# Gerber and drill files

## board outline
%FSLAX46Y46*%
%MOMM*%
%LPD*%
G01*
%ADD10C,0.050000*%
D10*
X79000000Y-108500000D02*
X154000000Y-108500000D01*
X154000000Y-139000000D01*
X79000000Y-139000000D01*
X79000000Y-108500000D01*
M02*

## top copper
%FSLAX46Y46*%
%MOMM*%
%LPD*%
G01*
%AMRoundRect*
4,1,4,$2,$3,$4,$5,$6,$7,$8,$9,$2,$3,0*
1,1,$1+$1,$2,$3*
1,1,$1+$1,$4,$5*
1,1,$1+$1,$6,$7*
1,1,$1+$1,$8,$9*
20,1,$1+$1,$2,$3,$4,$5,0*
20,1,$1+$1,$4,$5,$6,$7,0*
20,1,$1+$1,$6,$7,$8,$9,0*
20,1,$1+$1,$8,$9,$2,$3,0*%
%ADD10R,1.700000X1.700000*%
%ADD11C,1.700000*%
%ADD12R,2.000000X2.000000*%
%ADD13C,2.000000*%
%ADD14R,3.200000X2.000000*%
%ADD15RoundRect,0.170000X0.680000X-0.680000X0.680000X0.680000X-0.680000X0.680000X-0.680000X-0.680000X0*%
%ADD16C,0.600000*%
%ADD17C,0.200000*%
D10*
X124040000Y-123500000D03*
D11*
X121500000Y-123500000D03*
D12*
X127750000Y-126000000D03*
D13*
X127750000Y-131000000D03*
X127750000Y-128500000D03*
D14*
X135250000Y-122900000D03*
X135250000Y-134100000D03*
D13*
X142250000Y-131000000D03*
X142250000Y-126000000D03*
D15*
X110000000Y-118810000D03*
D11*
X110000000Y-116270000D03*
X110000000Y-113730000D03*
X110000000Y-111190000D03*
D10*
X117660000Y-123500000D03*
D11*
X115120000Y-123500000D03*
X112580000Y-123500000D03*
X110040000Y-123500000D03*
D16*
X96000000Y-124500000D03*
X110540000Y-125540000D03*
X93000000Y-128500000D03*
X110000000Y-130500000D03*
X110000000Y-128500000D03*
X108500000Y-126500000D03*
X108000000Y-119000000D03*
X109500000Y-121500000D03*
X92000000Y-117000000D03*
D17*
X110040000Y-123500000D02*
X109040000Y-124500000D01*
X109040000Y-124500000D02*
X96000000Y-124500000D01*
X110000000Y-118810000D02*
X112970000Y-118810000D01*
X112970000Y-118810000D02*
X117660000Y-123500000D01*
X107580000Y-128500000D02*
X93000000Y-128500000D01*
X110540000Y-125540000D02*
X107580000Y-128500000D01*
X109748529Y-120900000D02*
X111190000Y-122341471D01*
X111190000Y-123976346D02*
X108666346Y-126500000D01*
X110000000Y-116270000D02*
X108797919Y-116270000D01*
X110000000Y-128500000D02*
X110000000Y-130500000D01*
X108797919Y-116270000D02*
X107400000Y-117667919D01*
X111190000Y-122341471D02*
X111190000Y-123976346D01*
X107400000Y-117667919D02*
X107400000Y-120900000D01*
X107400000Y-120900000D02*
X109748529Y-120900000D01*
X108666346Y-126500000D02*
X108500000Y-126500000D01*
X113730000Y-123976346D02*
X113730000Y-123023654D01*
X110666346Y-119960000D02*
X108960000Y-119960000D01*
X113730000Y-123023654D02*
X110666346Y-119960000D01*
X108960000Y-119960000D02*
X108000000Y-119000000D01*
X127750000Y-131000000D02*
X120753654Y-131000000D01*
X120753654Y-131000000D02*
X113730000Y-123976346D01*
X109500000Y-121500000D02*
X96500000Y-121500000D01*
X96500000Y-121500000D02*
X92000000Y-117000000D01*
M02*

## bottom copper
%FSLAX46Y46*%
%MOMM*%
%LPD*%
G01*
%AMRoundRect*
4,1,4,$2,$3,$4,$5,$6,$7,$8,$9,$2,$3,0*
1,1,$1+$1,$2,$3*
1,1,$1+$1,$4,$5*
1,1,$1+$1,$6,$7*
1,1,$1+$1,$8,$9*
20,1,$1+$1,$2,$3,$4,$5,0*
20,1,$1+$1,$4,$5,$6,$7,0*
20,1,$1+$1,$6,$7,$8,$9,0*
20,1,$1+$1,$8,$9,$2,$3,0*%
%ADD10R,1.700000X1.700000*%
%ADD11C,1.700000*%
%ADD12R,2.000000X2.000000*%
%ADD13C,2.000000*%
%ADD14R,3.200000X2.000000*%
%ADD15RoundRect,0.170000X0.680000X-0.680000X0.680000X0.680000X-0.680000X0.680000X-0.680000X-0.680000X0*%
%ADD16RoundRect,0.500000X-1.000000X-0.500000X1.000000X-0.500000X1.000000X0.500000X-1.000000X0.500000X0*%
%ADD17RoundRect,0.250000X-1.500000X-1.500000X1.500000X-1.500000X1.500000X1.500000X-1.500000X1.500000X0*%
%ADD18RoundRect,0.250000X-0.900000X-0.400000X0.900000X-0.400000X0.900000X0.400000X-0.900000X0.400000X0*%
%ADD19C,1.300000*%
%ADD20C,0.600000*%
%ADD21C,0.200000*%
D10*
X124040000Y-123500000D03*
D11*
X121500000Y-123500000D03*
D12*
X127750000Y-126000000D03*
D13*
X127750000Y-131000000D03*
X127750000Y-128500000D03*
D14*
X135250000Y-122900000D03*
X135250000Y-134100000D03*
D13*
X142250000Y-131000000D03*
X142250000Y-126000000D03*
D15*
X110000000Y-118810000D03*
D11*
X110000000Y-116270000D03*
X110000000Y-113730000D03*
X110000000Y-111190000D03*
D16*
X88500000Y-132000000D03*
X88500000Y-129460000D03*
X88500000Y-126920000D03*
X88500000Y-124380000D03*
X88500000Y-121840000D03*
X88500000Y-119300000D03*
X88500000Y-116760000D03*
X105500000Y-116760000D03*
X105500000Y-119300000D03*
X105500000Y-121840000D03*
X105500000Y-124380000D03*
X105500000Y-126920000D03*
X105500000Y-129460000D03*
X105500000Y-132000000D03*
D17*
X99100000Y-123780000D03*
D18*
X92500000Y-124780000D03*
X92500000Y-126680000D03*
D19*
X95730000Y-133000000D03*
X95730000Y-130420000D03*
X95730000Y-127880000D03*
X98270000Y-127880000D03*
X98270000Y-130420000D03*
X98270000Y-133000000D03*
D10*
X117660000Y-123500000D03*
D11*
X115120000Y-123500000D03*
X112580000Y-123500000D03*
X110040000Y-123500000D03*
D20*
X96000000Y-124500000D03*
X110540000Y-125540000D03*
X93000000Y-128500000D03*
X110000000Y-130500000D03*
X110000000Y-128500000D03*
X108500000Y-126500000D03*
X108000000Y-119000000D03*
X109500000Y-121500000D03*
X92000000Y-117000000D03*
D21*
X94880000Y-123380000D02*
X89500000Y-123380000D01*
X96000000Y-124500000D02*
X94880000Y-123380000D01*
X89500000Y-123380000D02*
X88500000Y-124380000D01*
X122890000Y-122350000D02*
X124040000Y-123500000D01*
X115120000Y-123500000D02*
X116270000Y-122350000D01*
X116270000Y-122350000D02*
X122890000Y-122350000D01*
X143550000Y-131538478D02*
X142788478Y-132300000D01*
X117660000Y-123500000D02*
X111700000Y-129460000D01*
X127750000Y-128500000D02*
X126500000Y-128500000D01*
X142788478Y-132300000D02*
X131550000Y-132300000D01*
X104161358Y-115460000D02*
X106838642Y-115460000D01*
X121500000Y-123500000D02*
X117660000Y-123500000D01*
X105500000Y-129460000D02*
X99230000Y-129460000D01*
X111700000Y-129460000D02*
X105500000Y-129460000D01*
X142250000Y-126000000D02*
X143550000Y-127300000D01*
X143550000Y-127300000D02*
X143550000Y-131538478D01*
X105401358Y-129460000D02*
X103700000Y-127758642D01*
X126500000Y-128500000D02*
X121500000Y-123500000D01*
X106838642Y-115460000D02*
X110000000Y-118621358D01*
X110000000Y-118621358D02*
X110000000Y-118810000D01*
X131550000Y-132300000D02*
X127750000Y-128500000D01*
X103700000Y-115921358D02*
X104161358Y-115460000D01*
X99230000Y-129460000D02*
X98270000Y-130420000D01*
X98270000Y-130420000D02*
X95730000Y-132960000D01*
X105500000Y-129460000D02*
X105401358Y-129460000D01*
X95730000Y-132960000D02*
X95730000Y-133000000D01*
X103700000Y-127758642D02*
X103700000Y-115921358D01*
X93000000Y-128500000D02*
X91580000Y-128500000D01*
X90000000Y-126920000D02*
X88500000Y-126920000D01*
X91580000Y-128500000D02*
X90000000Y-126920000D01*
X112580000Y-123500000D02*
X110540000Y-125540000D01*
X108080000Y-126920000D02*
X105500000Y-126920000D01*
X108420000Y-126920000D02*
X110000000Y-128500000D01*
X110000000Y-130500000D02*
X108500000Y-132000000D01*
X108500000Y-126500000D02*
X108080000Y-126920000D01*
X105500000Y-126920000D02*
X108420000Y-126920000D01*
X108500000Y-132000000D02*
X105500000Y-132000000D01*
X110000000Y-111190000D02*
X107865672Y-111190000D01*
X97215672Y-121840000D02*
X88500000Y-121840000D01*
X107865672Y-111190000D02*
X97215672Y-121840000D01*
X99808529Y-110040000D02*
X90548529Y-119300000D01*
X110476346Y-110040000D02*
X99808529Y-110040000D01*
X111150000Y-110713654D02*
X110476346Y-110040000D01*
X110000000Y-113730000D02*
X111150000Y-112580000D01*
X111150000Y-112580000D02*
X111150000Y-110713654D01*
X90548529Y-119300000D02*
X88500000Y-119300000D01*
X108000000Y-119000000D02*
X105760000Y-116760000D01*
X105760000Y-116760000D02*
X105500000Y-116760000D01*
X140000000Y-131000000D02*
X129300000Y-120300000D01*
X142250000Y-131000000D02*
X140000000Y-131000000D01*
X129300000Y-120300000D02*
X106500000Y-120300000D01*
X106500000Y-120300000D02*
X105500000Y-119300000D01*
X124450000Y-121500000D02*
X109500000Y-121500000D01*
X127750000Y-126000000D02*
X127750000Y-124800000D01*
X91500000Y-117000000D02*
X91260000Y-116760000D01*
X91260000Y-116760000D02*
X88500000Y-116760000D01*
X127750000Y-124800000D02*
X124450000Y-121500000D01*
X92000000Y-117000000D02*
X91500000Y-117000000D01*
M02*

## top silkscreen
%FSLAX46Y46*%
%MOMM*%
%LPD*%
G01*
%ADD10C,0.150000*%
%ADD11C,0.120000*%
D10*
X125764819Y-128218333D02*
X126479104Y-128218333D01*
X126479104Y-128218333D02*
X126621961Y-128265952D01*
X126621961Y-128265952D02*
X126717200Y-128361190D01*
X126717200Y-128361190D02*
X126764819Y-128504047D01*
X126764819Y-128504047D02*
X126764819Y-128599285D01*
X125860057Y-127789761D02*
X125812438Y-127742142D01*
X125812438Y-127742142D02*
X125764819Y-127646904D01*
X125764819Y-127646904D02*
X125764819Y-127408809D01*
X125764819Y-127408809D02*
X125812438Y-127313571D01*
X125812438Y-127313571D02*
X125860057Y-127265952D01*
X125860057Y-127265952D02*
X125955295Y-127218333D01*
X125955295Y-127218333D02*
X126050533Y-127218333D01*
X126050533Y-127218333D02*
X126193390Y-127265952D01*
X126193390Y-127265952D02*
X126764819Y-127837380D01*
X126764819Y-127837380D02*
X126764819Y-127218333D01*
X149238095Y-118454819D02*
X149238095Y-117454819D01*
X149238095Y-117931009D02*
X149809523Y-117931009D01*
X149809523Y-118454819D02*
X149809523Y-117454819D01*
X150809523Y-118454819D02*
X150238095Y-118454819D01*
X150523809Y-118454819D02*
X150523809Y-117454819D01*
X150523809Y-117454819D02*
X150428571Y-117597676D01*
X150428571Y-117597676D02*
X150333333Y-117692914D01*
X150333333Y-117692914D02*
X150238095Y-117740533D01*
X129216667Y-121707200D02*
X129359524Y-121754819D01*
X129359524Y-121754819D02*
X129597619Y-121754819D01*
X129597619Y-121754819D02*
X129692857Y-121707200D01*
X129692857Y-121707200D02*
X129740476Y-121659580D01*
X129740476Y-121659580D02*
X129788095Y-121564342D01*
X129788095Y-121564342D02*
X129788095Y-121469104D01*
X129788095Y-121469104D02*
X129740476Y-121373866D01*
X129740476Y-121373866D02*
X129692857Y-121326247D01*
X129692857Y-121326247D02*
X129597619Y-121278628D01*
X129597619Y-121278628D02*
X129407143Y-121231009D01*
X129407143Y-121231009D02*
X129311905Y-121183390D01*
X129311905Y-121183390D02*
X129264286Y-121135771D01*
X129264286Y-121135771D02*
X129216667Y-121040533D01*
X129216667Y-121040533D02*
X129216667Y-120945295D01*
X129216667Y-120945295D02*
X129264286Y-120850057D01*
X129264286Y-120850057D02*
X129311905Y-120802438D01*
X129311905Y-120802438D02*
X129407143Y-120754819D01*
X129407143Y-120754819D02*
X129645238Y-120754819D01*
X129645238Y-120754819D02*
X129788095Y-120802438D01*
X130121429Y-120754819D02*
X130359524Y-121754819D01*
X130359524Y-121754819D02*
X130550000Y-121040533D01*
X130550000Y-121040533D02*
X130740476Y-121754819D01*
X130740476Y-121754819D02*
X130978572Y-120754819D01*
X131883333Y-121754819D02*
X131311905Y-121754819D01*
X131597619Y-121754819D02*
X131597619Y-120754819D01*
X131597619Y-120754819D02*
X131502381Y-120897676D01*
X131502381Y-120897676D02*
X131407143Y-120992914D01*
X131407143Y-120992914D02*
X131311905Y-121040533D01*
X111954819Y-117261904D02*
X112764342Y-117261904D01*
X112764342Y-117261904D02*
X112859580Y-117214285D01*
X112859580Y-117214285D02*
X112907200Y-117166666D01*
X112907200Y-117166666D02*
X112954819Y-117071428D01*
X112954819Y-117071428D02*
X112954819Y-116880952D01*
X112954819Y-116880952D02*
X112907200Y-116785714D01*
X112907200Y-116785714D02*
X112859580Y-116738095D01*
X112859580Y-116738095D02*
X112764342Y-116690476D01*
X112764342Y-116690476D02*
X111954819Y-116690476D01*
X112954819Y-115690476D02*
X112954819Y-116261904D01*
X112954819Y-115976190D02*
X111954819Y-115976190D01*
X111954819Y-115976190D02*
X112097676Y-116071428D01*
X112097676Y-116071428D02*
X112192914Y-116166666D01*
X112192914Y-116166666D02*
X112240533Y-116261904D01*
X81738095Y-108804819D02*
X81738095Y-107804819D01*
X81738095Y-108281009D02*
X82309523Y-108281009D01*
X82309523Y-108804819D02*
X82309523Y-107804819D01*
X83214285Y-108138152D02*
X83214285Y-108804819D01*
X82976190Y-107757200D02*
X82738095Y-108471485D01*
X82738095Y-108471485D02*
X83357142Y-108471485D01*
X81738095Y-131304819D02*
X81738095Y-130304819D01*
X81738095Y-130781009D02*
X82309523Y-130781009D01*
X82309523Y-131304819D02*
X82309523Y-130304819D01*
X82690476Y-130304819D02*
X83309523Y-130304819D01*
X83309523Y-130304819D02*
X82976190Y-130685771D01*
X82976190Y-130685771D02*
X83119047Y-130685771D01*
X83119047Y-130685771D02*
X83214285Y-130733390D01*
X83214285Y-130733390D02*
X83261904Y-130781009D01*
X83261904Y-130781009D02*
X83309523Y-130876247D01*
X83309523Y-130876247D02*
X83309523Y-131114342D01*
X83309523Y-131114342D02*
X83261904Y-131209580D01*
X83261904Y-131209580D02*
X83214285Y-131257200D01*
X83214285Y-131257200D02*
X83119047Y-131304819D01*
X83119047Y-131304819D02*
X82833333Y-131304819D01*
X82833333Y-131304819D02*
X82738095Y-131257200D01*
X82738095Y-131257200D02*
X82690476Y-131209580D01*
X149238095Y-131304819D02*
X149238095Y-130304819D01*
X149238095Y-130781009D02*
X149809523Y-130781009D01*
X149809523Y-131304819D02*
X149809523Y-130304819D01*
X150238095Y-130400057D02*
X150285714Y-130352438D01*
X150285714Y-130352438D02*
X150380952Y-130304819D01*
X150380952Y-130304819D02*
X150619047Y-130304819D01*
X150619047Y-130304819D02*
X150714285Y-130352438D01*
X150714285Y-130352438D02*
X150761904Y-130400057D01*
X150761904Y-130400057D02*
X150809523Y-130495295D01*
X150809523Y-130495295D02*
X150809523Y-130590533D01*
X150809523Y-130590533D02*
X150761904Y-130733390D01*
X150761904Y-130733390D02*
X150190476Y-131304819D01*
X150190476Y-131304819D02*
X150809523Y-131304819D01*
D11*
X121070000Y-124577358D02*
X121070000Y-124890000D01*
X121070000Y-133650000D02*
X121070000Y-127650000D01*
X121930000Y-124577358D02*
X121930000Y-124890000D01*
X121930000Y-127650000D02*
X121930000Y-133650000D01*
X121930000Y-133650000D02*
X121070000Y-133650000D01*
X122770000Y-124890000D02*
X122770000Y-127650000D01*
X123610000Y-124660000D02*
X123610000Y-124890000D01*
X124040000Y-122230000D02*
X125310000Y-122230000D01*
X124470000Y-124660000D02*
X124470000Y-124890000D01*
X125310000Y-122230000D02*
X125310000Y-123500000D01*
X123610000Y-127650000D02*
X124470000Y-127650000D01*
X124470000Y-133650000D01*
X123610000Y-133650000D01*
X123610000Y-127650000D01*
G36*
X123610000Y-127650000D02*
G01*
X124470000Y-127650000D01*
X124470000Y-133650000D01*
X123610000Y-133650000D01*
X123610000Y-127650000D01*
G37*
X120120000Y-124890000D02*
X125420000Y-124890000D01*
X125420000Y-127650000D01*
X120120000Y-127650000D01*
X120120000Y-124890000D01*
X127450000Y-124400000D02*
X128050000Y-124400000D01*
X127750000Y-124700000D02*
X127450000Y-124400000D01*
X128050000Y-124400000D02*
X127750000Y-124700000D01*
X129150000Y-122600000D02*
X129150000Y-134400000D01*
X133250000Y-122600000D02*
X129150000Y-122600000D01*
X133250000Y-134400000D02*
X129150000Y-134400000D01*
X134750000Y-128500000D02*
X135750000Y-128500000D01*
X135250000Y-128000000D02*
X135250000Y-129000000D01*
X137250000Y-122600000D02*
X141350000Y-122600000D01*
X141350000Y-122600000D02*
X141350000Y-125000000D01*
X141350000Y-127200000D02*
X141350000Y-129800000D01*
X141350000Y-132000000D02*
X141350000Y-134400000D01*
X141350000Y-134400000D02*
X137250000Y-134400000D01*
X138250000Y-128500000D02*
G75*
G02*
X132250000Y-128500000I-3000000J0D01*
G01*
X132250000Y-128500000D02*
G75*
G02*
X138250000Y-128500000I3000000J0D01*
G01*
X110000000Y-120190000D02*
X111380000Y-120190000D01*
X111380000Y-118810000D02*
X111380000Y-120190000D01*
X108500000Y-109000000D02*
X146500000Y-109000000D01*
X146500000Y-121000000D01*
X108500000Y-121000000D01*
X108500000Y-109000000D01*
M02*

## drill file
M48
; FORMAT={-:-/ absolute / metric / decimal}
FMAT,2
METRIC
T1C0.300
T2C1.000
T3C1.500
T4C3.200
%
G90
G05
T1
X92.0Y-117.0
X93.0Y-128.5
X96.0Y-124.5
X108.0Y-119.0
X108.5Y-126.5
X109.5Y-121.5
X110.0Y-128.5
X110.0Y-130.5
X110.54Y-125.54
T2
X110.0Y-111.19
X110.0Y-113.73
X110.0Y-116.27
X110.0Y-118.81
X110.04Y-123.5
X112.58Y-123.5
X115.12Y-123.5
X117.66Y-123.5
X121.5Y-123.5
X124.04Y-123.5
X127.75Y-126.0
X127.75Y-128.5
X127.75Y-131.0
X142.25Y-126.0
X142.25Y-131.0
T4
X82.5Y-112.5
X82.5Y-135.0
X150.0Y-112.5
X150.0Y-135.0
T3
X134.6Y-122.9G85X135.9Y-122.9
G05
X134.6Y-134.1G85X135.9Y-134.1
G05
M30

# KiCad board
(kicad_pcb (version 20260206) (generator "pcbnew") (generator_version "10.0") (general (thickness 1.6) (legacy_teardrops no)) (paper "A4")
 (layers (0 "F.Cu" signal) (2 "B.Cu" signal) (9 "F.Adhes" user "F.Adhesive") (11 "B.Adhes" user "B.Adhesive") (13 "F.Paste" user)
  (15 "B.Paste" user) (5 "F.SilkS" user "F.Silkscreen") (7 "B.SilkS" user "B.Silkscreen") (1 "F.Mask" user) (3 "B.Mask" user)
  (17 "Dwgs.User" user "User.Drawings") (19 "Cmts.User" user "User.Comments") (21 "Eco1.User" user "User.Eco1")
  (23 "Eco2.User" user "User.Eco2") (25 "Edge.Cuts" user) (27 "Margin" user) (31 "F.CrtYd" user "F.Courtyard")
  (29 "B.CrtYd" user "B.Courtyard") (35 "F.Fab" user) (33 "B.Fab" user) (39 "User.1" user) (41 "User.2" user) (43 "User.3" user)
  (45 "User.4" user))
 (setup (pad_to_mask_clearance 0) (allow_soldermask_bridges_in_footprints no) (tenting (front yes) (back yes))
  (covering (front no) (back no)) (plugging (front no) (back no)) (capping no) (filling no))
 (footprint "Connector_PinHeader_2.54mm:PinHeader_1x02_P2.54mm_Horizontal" (layer "F.Cu") (at 124.04 123.5 -90)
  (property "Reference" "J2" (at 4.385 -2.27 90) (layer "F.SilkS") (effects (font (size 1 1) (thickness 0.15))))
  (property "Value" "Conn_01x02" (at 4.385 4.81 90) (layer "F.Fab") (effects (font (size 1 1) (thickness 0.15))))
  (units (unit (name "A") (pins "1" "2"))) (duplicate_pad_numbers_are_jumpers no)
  (fp_line (start 1.077358 2.97) (end 1.39 2.97) (stroke (width 0.12) (type solid)) (layer "F.SilkS"))
  (fp_line (start 10.15 2.97) (end 4.15 2.97) (stroke (width 0.12) (type solid)) (layer "F.SilkS"))
  (fp_line (start 1.077358 2.11) (end 1.39 2.11) (stroke (width 0.12) (type solid)) (layer "F.SilkS"))
  (fp_line (start 4.15 2.11) (end 10.15 2.11) (stroke (width 0.12) (type solid)) (layer "F.SilkS"))
  (fp_line (start 10.15 2.11) (end 10.15 2.97) (stroke (width 0.12) (type solid)) (layer "F.SilkS"))
  (fp_line (start 1.39 1.27) (end 4.15 1.27) (stroke (width 0.12) (type solid)) (layer "F.SilkS"))
  (fp_line (start 1.16 0.43) (end 1.39 0.43) (stroke (width 0.12) (type solid)) (layer "F.SilkS"))
  (fp_line (start -1.27 0) (end -1.27 -1.27) (stroke (width 0.12) (type solid)) (layer "F.SilkS"))
  (fp_line (start 1.16 -0.43) (end 1.39 -0.43) (stroke (width 0.12) (type solid)) (layer "F.SilkS"))
  (fp_line (start -1.27 -1.27) (end 0 -1.27) (stroke (width 0.12) (type solid)) (layer "F.SilkS"))
  (fp_rect (start 4.15 -0.43) (end 10.15 0.43) (stroke (width 0.12) (type solid)) (fill yes) (layer "F.SilkS"))
  (fp_rect (start 1.39 -1.38) (end 4.15 3.92) (stroke (width 0.12) (type solid)) (fill no) (layer "F.SilkS"))
  (pad "1" thru_hole rect (at 0 0 270) (size 1.7 1.7) (drill 1) (layers "*.Cu" "*.Mask") (remove_unused_layers no) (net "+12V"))
  (pad "2" thru_hole circle (at 0 2.54 270) (size 1.7 1.7) (drill 1) (layers "*.Cu" "*.Mask") (remove_unused_layers no) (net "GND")))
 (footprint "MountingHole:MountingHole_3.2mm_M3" (layer "F.Cu") (at 150 112.5)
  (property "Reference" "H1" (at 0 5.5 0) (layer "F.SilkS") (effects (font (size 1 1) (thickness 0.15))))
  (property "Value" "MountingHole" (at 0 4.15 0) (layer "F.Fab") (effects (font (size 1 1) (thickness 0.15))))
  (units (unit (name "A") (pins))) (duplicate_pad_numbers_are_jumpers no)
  (pad "" np_thru_hole circle (at 0 0) (size 3.2 3.2) (drill 3.2) (layers "*.Cu" "*.Mask")))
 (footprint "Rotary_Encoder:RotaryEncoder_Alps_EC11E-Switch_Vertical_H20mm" (layer "F.Cu") (at 127.75 126)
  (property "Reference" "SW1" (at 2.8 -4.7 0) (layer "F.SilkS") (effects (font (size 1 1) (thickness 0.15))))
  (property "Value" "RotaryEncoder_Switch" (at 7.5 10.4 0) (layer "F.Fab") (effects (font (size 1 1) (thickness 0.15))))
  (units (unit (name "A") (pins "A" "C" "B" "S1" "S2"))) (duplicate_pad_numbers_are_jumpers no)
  (fp_line (start -0.3 -1.6) (end 0.3 -1.6) (stroke (width 0.12) (type solid)) (layer "F.SilkS"))
  (fp_line (start 0 -1.3) (end -0.3 -1.6) (stroke (width 0.12) (type solid)) (layer "F.SilkS"))
  (fp_line (start 0.3 -1.6) (end 0 -1.3) (stroke (width 0.12) (type solid)) (layer "F.SilkS"))
  (fp_line (start 1.4 -3.4) (end 1.4 8.4) (stroke (width 0.12) (type solid)) (layer "F.SilkS"))
  (fp_line (start 5.5 -3.4) (end 1.4 -3.4) (stroke (width 0.12) (type solid)) (layer "F.SilkS"))
  (fp_line (start 5.5 8.4) (end 1.4 8.4) (stroke (width 0.12) (type solid)) (layer "F.SilkS"))
  (fp_line (start 7 2.5) (end 8 2.5) (stroke (width 0.12) (type solid)) (layer "F.SilkS"))
  (fp_line (start 7.5 2) (end 7.5 3) (stroke (width 0.12) (type solid)) (layer "F.SilkS"))
  (fp_line (start 9.5 -3.4) (end 13.6 -3.4) (stroke (width 0.12) (type solid)) (layer "F.SilkS"))
  (fp_line (start 13.6 -3.4) (end 13.6 -1) (stroke (width 0.12) (type solid)) (layer "F.SilkS"))
  (fp_line (start 13.6 1.2) (end 13.6 3.8) (stroke (width 0.12) (type solid)) (layer "F.SilkS"))
  (fp_line (start 13.6 6) (end 13.6 8.4) (stroke (width 0.12) (type solid)) (layer "F.SilkS"))
  (fp_line (start 13.6 8.4) (end 9.5 8.4) (stroke (width 0.12) (type solid)) (layer "F.SilkS"))
  (fp_circle (center 7.5 2.5) (end 10.5 2.5) (stroke (width 0.12) (type solid)) (fill no) (layer "F.SilkS"))
  (pad "A" thru_hole rect (at 0 0) (size 2 2) (drill 1) (layers "*.Cu" "*.Mask") (remove_unused_layers no) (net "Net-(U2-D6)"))
  (pad "B" thru_hole circle (at 0 5) (size 2 2) (drill 1) (layers "*.Cu" "*.Mask") (remove_unused_layers no) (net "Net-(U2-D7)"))
  (pad "C" thru_hole circle (at 0 2.5) (size 2 2) (drill 1) (layers "*.Cu" "*.Mask") (remove_unused_layers no) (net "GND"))
  (pad "MP" thru_hole rect (at 7.5 -3.1) (size 3.2 2) (drill oval 2.8 1.5) (layers "*.Cu" "*.Mask") (remove_unused_layers no))
  (pad "MP" thru_hole rect (at 7.5 8.1) (size 3.2 2) (drill oval 2.8 1.5) (layers "*.Cu" "*.Mask") (remove_unused_layers no))
  (pad "S1" thru_hole circle (at 14.5 5) (size 2 2) (drill 1) (layers "*.Cu" "*.Mask") (remove_unused_layers no) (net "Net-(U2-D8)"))
  (pad "S2" thru_hole circle (at 14.5 0) (size 2 2) (drill 1) (layers "*.Cu" "*.Mask") (remove_unused_layers no) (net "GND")))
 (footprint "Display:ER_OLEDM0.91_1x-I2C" (layer "F.Cu") (at 110 118.81 90)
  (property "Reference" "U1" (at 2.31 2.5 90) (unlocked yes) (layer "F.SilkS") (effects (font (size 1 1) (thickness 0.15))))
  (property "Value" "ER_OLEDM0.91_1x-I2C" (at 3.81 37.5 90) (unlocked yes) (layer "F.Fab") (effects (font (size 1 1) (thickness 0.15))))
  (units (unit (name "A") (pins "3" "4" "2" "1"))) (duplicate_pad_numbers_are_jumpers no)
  (fp_line (start -1.38 0) (end -1.38 1.38) (stroke (width 0.12) (type solid)) (layer "F.SilkS"))
  (fp_line (start 0 1.38) (end -1.38 1.38) (stroke (width 0.12) (type solid)) (layer "F.SilkS"))
  (fp_rect (start -2.19 -1.5) (end 9.81 36.5) (stroke (width 0.12) (type solid)) (fill no) (layer "F.SilkS"))
  (pad "1" thru_hole roundrect (at 0 0 90) (size 1.7 1.7) (drill 1) (layers "*.Cu" "*.Mask") (remove_unused_layers no)
   (roundrect_rratio 0.1) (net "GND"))
  (pad "2" thru_hole circle (at 2.54 0 90) (size 1.7 1.7) (drill 1) (layers "*.Cu" "*.Mask") (remove_unused_layers no) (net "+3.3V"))
  (pad "3" thru_hole circle (at 5.08 0 90) (size 1.7 1.7) (drill 1) (layers "*.Cu" "*.Mask") (remove_unused_layers no) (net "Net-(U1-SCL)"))
  (pad "4" thru_hole circle (at 7.62 0 90) (size 1.7 1.7) (drill 1) (layers "*.Cu" "*.Mask") (remove_unused_layers no) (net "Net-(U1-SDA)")))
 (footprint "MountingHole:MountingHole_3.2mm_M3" (layer "F.Cu") (at 82.5 112.5)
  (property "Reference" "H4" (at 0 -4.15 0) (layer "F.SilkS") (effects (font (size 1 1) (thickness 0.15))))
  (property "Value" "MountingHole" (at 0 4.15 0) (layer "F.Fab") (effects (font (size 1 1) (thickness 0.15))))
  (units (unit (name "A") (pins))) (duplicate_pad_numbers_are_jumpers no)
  (pad "" np_thru_hole circle (at 0 0) (size 3.2 3.2) (drill 3.2) (layers "*.Cu" "*.Mask")))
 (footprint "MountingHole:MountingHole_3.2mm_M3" (layer "F.Cu") (at 82.5 135)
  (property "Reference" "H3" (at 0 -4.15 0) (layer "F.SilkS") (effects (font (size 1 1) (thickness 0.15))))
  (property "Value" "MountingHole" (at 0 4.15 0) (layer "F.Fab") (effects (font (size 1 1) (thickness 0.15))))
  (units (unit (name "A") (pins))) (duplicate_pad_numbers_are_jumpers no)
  (pad "" np_thru_hole circle (at 0 0) (size 3.2 3.2) (drill 3.2) (layers "*.Cu" "*.Mask")))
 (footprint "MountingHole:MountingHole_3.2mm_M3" (layer "F.Cu") (at 150 135)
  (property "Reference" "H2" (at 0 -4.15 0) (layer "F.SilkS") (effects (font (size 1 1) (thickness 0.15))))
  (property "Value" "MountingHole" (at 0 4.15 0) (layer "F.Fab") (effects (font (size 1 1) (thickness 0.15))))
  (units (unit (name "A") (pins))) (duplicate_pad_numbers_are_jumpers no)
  (pad "" np_thru_hole circle (at 0 0) (size 3.2 3.2) (drill 3.2) (layers "*.Cu" "*.Mask")))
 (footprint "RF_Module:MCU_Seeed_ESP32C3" (layer "B.Cu") (at 97 124.38)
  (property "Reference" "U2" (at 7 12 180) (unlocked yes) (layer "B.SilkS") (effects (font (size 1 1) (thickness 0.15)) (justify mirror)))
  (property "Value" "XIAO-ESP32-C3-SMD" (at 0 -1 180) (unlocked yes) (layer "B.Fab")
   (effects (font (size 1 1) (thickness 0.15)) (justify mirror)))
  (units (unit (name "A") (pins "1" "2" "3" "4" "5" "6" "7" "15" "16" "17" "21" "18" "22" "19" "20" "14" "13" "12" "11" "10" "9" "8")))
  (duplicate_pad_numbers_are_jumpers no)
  (pad "" smd roundrect (at 1.1 -1.6) (size 1.5 1.5) (layers "B.Paste") (roundrect_rratio 0.1666666667))
  (pad "" smd roundrect (at 1.1 0.4) (size 1.5 1.5) (layers "B.Paste") (roundrect_rratio 0.1666666667))
  (pad "" smd roundrect (at 3.1 -1.6) (size 1.5 1.5) (layers "B.Paste") (roundrect_rratio 0.1666666667))
  (pad "" smd roundrect (at 3.1 0.4) (size 1.5 1.5) (layers "B.Paste") (roundrect_rratio 0.1666666667))
  (pad "1" smd roundrect (at -8.5 7.62) (size 3 2) (layers "B.Cu" "B.Mask" "B.Paste") (roundrect_rratio 0.25)
   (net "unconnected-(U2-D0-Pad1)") (thermal_bridge_angle 45))
  (pad "2" smd roundrect (at -8.5 5.08) (size 3 2) (layers "B.Cu" "B.Mask" "B.Paste") (roundrect_rratio 0.25)
   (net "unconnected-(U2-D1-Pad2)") (thermal_bridge_angle 45))
  (pad "3" smd roundrect (at -8.5 2.54) (size 3 2) (layers "B.Cu" "B.Mask" "B.Paste") (roundrect_rratio 0.25) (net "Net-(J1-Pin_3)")
   (thermal_bridge_angle 45))
  (pad "4" smd roundrect (at -8.5 0) (size 3 2) (layers "B.Cu" "B.Mask" "B.Paste") (roundrect_rratio 0.25) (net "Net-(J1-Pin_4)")
   (thermal_bridge_angle 45))
  (pad "5" smd roundrect (at -8.5 -2.54) (size 3 2) (layers "B.Cu" "B.Mask" "B.Paste") (roundrect_rratio 0.25) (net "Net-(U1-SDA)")
   (thermal_bridge_angle 45))
  (pad "6" smd roundrect (at -8.5 -5.08) (size 3 2) (layers "B.Cu" "B.Mask" "B.Paste") (roundrect_rratio 0.25) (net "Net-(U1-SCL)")
   (thermal_bridge_angle 45))
  (pad "7" smd roundrect (at -8.5 -7.62) (size 3 2) (layers "B.Cu" "B.Mask" "B.Paste") (roundrect_rratio 0.25) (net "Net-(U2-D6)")
   (thermal_bridge_angle 45))
  (pad "8" smd roundrect (at 8.5 -7.62) (size 3 2) (layers "B.Cu" "B.Mask" "B.Paste") (roundrect_rratio 0.25) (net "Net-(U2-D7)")
   (thermal_bridge_angle 45))
  (pad "9" smd roundrect (at 8.5 -5.08) (size 3 2) (layers "B.Cu" "B.Mask" "B.Paste") (roundrect_rratio 0.25) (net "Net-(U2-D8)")
   (thermal_bridge_angle 45))
  (pad "10" smd roundrect (at 8.5 -2.54) (size 3 2) (layers "B.Cu" "B.Mask" "B.Paste") (roundrect_rratio 0.25)
   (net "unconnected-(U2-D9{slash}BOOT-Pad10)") (thermal_bridge_angle 45))
  (pad "11" smd roundrect (at 8.5 0) (size 3 2) (layers "B.Cu" "B.Mask" "B.Paste") (roundrect_rratio 0.25)
   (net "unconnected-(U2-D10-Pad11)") (thermal_bridge_angle 45))
  (pad "12" smd roundrect (at 8.5 2.54) (size 3 2) (layers "B.Cu" "B.Mask" "B.Paste") (roundrect_rratio 0.25) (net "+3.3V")
   (thermal_bridge_angle 45))
  (pad "13" smd roundrect (at 8.5 5.08) (size 3 2) (layers "B.Cu" "B.Mask" "B.Paste") (roundrect_rratio 0.25) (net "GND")
   (thermal_bridge_angle 45))
  (pad "14" smd roundrect (at 8.5 7.62) (size 3 2) (layers "B.Cu" "B.Mask" "B.Paste") (roundrect_rratio 0.25) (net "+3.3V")
   (thermal_bridge_angle 45))
  (pad "15" smd roundrect (at 2.1 -0.6) (size 3.5 3.5) (layers "B.Cu" "B.Mask") (roundrect_rratio 0.07142857143)
   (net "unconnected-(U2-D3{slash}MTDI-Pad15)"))
  (pad "16" smd roundrect (at -4.5 0.4) (size 2.3 1.3) (layers "B.Cu" "B.Mask" "B.Paste") (roundrect_rratio 0.1923076923)
   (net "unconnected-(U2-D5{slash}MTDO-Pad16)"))
  (pad "17" smd roundrect (at -4.5 2.3) (size 2.3 1.3) (layers "B.Cu" "B.Mask" "B.Paste") (roundrect_rratio 0.1923076923)
   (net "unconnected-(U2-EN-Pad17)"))
  (pad "18" smd circle (at -1.27 8.62) (size 1.3 1.3) (layers "B.Cu" "B.Mask" "B.Paste") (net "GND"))
  (pad "19" smd circle (at -1.27 6.04) (size 1.3 1.3) (layers "B.Cu" "B.Mask" "B.Paste") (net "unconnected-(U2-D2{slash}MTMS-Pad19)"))
  (pad "20" smd circle (at -1.27 3.5) (size 1.3 1.3) (layers "B.Cu" "B.Mask" "B.Paste") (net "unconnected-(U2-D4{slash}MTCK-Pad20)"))
  (pad "21" smd circle (at 1.27 3.5) (size 1.3 1.3) (layers "B.Cu" "B.Mask" "B.Paste") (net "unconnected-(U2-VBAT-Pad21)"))
  (pad "22" smd circle (at 1.27 6.04) (size 1.3 1.3) (layers "B.Cu" "B.Mask" "B.Paste") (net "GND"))
  (pad "23" smd circle (at 1.27 8.62) (size 1.3 1.3) (layers "B.Cu" "B.Mask" "B.Paste")))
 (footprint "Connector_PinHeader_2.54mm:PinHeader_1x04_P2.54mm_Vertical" (layer "B.Cu") (at 117.66 123.5 90)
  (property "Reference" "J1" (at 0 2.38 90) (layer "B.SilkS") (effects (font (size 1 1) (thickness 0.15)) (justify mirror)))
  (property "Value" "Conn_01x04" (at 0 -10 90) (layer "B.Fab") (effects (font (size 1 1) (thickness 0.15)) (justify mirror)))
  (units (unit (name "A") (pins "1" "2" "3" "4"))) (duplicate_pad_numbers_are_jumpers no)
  (pad "1" thru_hole rect (at 0 0 90) (size 1.7 1.7) (drill 1) (layers "*.Cu" "*.Mask") (remove_unused_layers no) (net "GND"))
  (pad "2" thru_hole circle (at 0 -2.54 90) (size 1.7 1.7) (drill 1) (layers "*.Cu" "*.Mask") (remove_unused_layers no) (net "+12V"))
  (pad "3" thru_hole circle (at 0 -5.08 90) (size 1.7 1.7) (drill 1) (layers "*.Cu" "*.Mask") (remove_unused_layers no)
   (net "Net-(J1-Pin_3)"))
  (pad "4" thru_hole circle (at 0 -7.62 90) (size 1.7 1.7) (drill 1) (layers "*.Cu" "*.Mask") (remove_unused_layers no)
   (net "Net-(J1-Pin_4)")))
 (gr_rect (start 79 108.5) (end 154 139) (stroke (width 0.05) (type default)) (fill no) (layer "Edge.Cuts"))
 (segment (start 110.04 123.5) (end 109.04 124.5) (width 0.2) (layer "F.Cu") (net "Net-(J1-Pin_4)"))
 (segment (start 109.04 124.5) (end 96 124.5) (width 0.2) (layer "F.Cu") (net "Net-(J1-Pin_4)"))
 (via (at 96 124.5) (size 0.6) (drill 0.3) (layers "F.Cu" "B.Cu") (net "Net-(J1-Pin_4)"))
 (segment (start 94.88 123.38) (end 89.5 123.38) (width 0.2) (layer "B.Cu") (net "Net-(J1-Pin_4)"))
 (segment (start 96 124.5) (end 94.88 123.38) (width 0.2) (layer "B.Cu") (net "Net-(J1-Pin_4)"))
 (segment (start 89.5 123.38) (end 88.5 124.38) (width 0.2) (layer "B.Cu") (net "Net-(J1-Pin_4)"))
 (segment (start 122.89 122.35) (end 124.04 123.5) (width 0.2) (layer "B.Cu") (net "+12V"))
 (segment (start 115.12 123.5) (end 116.27 122.35) (width 0.2) (layer "B.Cu") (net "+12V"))
 (segment (start 116.27 122.35) (end 122.89 122.35) (width 0.2) (layer "B.Cu") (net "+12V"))
 (segment (start 110 118.81) (end 112.97 118.81) (width 0.2) (layer "F.Cu") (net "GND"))
 (segment (start 112.97 118.81) (end 117.66 123.5) (width 0.2) (layer "F.Cu") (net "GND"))
 (segment (start 143.55 131.538478) (end 142.788478 132.3) (width 0.2) (layer "B.Cu") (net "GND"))
 (segment (start 117.66 123.5) (end 111.7 129.46) (width 0.2) (layer "B.Cu") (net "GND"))
 (segment (start 127.75 128.5) (end 126.5 128.5) (width 0.2) (layer "B.Cu") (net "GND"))
 (segment (start 142.788478 132.3) (end 131.55 132.3) (width 0.2) (layer "B.Cu") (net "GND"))
 (segment (start 104.161358 115.46) (end 106.838642 115.46) (width 0.2) (layer "B.Cu") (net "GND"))
 (segment (start 121.5 123.5) (end 117.66 123.5) (width 0.2) (layer "B.Cu") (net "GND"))
 (segment (start 105.5 129.46) (end 99.23 129.46) (width 0.2) (layer "B.Cu") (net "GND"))
 (segment (start 111.7 129.46) (end 105.5 129.46) (width 0.2) (layer "B.Cu") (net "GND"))
 (segment (start 142.25 126) (end 143.55 127.3) (width 0.2) (layer "B.Cu") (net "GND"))
 (segment (start 143.55 127.3) (end 143.55 131.538478) (width 0.2) (layer "B.Cu") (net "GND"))
 (segment (start 105.401358 129.46) (end 103.7 127.758642) (width 0.2) (layer "B.Cu") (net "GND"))
 (segment (start 126.5 128.5) (end 121.5 123.5) (width 0.2) (layer "B.Cu") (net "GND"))
 (segment (start 106.838642 115.46) (end 110 118.621358) (width 0.2) (layer "B.Cu") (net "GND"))
 (segment (start 110 118.621358) (end 110 118.81) (width 0.2) (layer "B.Cu") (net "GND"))
 (segment (start 131.55 132.3) (end 127.75 128.5) (width 0.2) (layer "B.Cu") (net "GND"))
 (segment (start 103.7 115.921358) (end 104.161358 115.46) (width 0.2) (layer "B.Cu") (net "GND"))
 (segment (start 99.23 129.46) (end 98.27 130.42) (width 0.2) (layer "B.Cu") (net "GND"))
 (segment (start 98.27 130.42) (end 95.73 132.96) (width 0.2) (layer "B.Cu") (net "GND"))
 (segment (start 105.5 129.46) (end 105.401358 129.46) (width 0.2) (layer "B.Cu") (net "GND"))
 (segment (start 95.73 132.96) (end 95.73 133) (width 0.2) (layer "B.Cu") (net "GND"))
 (segment (start 103.7 127.758642) (end 103.7 115.921358) (width 0.2) (layer "B.Cu") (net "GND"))
 (segment (start 107.58 128.5) (end 93 128.5) (width 0.2) (layer "F.Cu") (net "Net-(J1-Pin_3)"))
 (segment (start 110.54 125.54) (end 107.58 128.5) (width 0.2) (layer "F.Cu") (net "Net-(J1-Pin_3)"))
 (via (at 110.54 125.54) (size 0.6) (drill 0.3) (layers "F.Cu" "B.Cu") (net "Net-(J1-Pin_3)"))
 (via (at 93 128.5) (size 0.6) (drill 0.3) (layers "F.Cu" "B.Cu") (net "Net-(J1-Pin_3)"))
 (segment (start 93 128.5) (end 91.58 128.5) (width 0.2) (layer "B.Cu") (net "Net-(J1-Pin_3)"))
 (segment (start 90 126.92) (end 88.5 126.92) (width 0.2) (layer "B.Cu") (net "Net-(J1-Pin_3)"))
 (segment (start 91.58 128.5) (end 90 126.92) (width 0.2) (layer "B.Cu") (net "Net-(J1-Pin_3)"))
 (segment (start 112.58 123.5) (end 110.54 125.54) (width 0.2) (layer "B.Cu") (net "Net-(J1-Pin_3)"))
 (segment (start 109.748529 120.9) (end 111.19 122.341471) (width 0.2) (layer "F.Cu") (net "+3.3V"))
 (segment (start 111.19 123.976346) (end 108.666346 126.5) (width 0.2) (layer "F.Cu") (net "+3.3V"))
 (segment (start 110 116.27) (end 108.797919 116.27) (width 0.2) (layer "F.Cu") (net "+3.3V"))
 (segment (start 110 128.5) (end 110 130.5) (width 0.2) (layer "F.Cu") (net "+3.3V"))
 (segment (start 108.797919 116.27) (end 107.4 117.667919) (width 0.2) (layer "F.Cu") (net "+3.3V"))
 (segment (start 111.19 122.341471) (end 111.19 123.976346) (width 0.2) (layer "F.Cu") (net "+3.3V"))
 (segment (start 107.4 117.667919) (end 107.4 120.9) (width 0.2) (layer "F.Cu") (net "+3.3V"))
 (segment (start 107.4 120.9) (end 109.748529 120.9) (width 0.2) (layer "F.Cu") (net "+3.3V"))
 (segment (start 108.666346 126.5) (end 108.5 126.5) (width 0.2) (layer "F.Cu") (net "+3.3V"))
 (via (at 110 130.5) (size 0.6) (drill 0.3) (layers "F.Cu" "B.Cu") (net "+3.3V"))
 (via (at 110 128.5) (size 0.6) (drill 0.3) (layers "F.Cu" "B.Cu") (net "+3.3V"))
 (via (at 108.5 126.5) (size 0.6) (drill 0.3) (layers "F.Cu" "B.Cu") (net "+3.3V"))
 (segment (start 108.08 126.92) (end 105.5 126.92) (width 0.2) (layer "B.Cu") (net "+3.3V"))
 (segment (start 108.42 126.92) (end 110 128.5) (width 0.2) (layer "B.Cu") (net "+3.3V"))
 (segment (start 110 130.5) (end 108.5 132) (width 0.2) (layer "B.Cu") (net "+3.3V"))
 (segment (start 108.5 126.5) (end 108.08 126.92) (width 0.2) (layer "B.Cu") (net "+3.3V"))
 (segment (start 105.5 126.92) (end 108.42 126.92) (width 0.2) (layer "B.Cu") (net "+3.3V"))
 (segment (start 108.5 132) (end 105.5 132) (width 0.2) (layer "B.Cu") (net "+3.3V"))
 (segment (start 110 111.19) (end 107.865672 111.19) (width 0.2) (layer "B.Cu") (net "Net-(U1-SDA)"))
 (segment (start 97.215672 121.84) (end 88.5 121.84) (width 0.2) (layer "B.Cu") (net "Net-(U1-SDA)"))
 (segment (start 107.865672 111.19) (end 97.215672 121.84) (width 0.2) (layer "B.Cu") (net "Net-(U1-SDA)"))
 (segment (start 99.808529 110.04) (end 90.548529 119.3) (width 0.2) (layer "B.Cu") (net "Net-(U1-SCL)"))
 (segment (start 110.476346 110.04) (end 99.808529 110.04) (width 0.2) (layer "B.Cu") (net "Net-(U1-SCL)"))
 (segment (start 111.15 110.713654) (end 110.476346 110.04) (width 0.2) (layer "B.Cu") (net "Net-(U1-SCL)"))
 (segment (start 110 113.73) (end 111.15 112.58) (width 0.2) (layer "B.Cu") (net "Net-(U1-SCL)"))
 (segment (start 111.15 112.58) (end 111.15 110.713654) (width 0.2) (layer "B.Cu") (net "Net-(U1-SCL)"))
 (segment (start 90.548529 119.3) (end 88.5 119.3) (width 0.2) (layer "B.Cu") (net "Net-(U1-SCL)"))
 (segment (start 113.73 123.976346) (end 113.73 123.023654) (width 0.2) (layer "F.Cu") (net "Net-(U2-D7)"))
 (segment (start 110.666346 119.96) (end 108.96 119.96) (width 0.2) (layer "F.Cu") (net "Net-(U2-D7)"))
 (segment (start 113.73 123.023654) (end 110.666346 119.96) (width 0.2) (layer "F.Cu") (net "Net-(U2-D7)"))
 (segment (start 108.96 119.96) (end 108 119) (width 0.2) (layer "F.Cu") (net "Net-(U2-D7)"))
 (segment (start 127.75 131) (end 120.753654 131) (width 0.2) (layer "F.Cu") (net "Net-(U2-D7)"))
 (segment (start 120.753654 131) (end 113.73 123.976346) (width 0.2) (layer "F.Cu") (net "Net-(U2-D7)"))
 (via (at 108 119) (size 0.6) (drill 0.3) (layers "F.Cu" "B.Cu") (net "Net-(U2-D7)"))
 (segment (start 108 119) (end 105.76 116.76) (width 0.2) (layer "B.Cu") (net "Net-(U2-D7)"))
 (segment (start 105.76 116.76) (end 105.5 116.76) (width 0.2) (layer "B.Cu") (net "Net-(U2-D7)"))
 (segment (start 140 131) (end 129.3 120.3) (width 0.2) (layer "B.Cu") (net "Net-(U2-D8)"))
 (segment (start 142.25 131) (end 140 131) (width 0.2) (layer "B.Cu") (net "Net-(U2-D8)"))
 (segment (start 129.3 120.3) (end 106.5 120.3) (width 0.2) (layer "B.Cu") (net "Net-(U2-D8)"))
 (segment (start 106.5 120.3) (end 105.5 119.3) (width 0.2) (layer "B.Cu") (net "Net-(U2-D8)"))
 (segment (start 109.5 121.5) (end 96.5 121.5) (width 0.2) (layer "F.Cu") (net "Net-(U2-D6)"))
 (segment (start 96.5 121.5) (end 92 117) (width 0.2) (layer "F.Cu") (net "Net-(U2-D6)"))
 (via (at 109.5 121.5) (size 0.6) (drill 0.3) (layers "F.Cu" "B.Cu") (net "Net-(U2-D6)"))
 (via (at 92 117) (size 0.6) (drill 0.3) (layers "F.Cu" "B.Cu") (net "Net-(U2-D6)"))
 (segment (start 124.45 121.5) (end 109.5 121.5) (width 0.2) (layer "B.Cu") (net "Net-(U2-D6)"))
 (segment (start 127.75 126) (end 127.75 124.8) (width 0.2) (layer "B.Cu") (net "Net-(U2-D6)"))
 (segment (start 91.5 117) (end 91.26 116.76) (width 0.2) (layer "B.Cu") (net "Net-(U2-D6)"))
 (segment (start 91.26 116.76) (end 88.5 116.76) (width 0.2) (layer "B.Cu") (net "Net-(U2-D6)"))
 (segment (start 127.75 124.8) (end 124.45 121.5) (width 0.2) (layer "B.Cu") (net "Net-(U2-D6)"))
 (segment (start 92 117) (end 91.5 117) (width 0.2) (layer "B.Cu") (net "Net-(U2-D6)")))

